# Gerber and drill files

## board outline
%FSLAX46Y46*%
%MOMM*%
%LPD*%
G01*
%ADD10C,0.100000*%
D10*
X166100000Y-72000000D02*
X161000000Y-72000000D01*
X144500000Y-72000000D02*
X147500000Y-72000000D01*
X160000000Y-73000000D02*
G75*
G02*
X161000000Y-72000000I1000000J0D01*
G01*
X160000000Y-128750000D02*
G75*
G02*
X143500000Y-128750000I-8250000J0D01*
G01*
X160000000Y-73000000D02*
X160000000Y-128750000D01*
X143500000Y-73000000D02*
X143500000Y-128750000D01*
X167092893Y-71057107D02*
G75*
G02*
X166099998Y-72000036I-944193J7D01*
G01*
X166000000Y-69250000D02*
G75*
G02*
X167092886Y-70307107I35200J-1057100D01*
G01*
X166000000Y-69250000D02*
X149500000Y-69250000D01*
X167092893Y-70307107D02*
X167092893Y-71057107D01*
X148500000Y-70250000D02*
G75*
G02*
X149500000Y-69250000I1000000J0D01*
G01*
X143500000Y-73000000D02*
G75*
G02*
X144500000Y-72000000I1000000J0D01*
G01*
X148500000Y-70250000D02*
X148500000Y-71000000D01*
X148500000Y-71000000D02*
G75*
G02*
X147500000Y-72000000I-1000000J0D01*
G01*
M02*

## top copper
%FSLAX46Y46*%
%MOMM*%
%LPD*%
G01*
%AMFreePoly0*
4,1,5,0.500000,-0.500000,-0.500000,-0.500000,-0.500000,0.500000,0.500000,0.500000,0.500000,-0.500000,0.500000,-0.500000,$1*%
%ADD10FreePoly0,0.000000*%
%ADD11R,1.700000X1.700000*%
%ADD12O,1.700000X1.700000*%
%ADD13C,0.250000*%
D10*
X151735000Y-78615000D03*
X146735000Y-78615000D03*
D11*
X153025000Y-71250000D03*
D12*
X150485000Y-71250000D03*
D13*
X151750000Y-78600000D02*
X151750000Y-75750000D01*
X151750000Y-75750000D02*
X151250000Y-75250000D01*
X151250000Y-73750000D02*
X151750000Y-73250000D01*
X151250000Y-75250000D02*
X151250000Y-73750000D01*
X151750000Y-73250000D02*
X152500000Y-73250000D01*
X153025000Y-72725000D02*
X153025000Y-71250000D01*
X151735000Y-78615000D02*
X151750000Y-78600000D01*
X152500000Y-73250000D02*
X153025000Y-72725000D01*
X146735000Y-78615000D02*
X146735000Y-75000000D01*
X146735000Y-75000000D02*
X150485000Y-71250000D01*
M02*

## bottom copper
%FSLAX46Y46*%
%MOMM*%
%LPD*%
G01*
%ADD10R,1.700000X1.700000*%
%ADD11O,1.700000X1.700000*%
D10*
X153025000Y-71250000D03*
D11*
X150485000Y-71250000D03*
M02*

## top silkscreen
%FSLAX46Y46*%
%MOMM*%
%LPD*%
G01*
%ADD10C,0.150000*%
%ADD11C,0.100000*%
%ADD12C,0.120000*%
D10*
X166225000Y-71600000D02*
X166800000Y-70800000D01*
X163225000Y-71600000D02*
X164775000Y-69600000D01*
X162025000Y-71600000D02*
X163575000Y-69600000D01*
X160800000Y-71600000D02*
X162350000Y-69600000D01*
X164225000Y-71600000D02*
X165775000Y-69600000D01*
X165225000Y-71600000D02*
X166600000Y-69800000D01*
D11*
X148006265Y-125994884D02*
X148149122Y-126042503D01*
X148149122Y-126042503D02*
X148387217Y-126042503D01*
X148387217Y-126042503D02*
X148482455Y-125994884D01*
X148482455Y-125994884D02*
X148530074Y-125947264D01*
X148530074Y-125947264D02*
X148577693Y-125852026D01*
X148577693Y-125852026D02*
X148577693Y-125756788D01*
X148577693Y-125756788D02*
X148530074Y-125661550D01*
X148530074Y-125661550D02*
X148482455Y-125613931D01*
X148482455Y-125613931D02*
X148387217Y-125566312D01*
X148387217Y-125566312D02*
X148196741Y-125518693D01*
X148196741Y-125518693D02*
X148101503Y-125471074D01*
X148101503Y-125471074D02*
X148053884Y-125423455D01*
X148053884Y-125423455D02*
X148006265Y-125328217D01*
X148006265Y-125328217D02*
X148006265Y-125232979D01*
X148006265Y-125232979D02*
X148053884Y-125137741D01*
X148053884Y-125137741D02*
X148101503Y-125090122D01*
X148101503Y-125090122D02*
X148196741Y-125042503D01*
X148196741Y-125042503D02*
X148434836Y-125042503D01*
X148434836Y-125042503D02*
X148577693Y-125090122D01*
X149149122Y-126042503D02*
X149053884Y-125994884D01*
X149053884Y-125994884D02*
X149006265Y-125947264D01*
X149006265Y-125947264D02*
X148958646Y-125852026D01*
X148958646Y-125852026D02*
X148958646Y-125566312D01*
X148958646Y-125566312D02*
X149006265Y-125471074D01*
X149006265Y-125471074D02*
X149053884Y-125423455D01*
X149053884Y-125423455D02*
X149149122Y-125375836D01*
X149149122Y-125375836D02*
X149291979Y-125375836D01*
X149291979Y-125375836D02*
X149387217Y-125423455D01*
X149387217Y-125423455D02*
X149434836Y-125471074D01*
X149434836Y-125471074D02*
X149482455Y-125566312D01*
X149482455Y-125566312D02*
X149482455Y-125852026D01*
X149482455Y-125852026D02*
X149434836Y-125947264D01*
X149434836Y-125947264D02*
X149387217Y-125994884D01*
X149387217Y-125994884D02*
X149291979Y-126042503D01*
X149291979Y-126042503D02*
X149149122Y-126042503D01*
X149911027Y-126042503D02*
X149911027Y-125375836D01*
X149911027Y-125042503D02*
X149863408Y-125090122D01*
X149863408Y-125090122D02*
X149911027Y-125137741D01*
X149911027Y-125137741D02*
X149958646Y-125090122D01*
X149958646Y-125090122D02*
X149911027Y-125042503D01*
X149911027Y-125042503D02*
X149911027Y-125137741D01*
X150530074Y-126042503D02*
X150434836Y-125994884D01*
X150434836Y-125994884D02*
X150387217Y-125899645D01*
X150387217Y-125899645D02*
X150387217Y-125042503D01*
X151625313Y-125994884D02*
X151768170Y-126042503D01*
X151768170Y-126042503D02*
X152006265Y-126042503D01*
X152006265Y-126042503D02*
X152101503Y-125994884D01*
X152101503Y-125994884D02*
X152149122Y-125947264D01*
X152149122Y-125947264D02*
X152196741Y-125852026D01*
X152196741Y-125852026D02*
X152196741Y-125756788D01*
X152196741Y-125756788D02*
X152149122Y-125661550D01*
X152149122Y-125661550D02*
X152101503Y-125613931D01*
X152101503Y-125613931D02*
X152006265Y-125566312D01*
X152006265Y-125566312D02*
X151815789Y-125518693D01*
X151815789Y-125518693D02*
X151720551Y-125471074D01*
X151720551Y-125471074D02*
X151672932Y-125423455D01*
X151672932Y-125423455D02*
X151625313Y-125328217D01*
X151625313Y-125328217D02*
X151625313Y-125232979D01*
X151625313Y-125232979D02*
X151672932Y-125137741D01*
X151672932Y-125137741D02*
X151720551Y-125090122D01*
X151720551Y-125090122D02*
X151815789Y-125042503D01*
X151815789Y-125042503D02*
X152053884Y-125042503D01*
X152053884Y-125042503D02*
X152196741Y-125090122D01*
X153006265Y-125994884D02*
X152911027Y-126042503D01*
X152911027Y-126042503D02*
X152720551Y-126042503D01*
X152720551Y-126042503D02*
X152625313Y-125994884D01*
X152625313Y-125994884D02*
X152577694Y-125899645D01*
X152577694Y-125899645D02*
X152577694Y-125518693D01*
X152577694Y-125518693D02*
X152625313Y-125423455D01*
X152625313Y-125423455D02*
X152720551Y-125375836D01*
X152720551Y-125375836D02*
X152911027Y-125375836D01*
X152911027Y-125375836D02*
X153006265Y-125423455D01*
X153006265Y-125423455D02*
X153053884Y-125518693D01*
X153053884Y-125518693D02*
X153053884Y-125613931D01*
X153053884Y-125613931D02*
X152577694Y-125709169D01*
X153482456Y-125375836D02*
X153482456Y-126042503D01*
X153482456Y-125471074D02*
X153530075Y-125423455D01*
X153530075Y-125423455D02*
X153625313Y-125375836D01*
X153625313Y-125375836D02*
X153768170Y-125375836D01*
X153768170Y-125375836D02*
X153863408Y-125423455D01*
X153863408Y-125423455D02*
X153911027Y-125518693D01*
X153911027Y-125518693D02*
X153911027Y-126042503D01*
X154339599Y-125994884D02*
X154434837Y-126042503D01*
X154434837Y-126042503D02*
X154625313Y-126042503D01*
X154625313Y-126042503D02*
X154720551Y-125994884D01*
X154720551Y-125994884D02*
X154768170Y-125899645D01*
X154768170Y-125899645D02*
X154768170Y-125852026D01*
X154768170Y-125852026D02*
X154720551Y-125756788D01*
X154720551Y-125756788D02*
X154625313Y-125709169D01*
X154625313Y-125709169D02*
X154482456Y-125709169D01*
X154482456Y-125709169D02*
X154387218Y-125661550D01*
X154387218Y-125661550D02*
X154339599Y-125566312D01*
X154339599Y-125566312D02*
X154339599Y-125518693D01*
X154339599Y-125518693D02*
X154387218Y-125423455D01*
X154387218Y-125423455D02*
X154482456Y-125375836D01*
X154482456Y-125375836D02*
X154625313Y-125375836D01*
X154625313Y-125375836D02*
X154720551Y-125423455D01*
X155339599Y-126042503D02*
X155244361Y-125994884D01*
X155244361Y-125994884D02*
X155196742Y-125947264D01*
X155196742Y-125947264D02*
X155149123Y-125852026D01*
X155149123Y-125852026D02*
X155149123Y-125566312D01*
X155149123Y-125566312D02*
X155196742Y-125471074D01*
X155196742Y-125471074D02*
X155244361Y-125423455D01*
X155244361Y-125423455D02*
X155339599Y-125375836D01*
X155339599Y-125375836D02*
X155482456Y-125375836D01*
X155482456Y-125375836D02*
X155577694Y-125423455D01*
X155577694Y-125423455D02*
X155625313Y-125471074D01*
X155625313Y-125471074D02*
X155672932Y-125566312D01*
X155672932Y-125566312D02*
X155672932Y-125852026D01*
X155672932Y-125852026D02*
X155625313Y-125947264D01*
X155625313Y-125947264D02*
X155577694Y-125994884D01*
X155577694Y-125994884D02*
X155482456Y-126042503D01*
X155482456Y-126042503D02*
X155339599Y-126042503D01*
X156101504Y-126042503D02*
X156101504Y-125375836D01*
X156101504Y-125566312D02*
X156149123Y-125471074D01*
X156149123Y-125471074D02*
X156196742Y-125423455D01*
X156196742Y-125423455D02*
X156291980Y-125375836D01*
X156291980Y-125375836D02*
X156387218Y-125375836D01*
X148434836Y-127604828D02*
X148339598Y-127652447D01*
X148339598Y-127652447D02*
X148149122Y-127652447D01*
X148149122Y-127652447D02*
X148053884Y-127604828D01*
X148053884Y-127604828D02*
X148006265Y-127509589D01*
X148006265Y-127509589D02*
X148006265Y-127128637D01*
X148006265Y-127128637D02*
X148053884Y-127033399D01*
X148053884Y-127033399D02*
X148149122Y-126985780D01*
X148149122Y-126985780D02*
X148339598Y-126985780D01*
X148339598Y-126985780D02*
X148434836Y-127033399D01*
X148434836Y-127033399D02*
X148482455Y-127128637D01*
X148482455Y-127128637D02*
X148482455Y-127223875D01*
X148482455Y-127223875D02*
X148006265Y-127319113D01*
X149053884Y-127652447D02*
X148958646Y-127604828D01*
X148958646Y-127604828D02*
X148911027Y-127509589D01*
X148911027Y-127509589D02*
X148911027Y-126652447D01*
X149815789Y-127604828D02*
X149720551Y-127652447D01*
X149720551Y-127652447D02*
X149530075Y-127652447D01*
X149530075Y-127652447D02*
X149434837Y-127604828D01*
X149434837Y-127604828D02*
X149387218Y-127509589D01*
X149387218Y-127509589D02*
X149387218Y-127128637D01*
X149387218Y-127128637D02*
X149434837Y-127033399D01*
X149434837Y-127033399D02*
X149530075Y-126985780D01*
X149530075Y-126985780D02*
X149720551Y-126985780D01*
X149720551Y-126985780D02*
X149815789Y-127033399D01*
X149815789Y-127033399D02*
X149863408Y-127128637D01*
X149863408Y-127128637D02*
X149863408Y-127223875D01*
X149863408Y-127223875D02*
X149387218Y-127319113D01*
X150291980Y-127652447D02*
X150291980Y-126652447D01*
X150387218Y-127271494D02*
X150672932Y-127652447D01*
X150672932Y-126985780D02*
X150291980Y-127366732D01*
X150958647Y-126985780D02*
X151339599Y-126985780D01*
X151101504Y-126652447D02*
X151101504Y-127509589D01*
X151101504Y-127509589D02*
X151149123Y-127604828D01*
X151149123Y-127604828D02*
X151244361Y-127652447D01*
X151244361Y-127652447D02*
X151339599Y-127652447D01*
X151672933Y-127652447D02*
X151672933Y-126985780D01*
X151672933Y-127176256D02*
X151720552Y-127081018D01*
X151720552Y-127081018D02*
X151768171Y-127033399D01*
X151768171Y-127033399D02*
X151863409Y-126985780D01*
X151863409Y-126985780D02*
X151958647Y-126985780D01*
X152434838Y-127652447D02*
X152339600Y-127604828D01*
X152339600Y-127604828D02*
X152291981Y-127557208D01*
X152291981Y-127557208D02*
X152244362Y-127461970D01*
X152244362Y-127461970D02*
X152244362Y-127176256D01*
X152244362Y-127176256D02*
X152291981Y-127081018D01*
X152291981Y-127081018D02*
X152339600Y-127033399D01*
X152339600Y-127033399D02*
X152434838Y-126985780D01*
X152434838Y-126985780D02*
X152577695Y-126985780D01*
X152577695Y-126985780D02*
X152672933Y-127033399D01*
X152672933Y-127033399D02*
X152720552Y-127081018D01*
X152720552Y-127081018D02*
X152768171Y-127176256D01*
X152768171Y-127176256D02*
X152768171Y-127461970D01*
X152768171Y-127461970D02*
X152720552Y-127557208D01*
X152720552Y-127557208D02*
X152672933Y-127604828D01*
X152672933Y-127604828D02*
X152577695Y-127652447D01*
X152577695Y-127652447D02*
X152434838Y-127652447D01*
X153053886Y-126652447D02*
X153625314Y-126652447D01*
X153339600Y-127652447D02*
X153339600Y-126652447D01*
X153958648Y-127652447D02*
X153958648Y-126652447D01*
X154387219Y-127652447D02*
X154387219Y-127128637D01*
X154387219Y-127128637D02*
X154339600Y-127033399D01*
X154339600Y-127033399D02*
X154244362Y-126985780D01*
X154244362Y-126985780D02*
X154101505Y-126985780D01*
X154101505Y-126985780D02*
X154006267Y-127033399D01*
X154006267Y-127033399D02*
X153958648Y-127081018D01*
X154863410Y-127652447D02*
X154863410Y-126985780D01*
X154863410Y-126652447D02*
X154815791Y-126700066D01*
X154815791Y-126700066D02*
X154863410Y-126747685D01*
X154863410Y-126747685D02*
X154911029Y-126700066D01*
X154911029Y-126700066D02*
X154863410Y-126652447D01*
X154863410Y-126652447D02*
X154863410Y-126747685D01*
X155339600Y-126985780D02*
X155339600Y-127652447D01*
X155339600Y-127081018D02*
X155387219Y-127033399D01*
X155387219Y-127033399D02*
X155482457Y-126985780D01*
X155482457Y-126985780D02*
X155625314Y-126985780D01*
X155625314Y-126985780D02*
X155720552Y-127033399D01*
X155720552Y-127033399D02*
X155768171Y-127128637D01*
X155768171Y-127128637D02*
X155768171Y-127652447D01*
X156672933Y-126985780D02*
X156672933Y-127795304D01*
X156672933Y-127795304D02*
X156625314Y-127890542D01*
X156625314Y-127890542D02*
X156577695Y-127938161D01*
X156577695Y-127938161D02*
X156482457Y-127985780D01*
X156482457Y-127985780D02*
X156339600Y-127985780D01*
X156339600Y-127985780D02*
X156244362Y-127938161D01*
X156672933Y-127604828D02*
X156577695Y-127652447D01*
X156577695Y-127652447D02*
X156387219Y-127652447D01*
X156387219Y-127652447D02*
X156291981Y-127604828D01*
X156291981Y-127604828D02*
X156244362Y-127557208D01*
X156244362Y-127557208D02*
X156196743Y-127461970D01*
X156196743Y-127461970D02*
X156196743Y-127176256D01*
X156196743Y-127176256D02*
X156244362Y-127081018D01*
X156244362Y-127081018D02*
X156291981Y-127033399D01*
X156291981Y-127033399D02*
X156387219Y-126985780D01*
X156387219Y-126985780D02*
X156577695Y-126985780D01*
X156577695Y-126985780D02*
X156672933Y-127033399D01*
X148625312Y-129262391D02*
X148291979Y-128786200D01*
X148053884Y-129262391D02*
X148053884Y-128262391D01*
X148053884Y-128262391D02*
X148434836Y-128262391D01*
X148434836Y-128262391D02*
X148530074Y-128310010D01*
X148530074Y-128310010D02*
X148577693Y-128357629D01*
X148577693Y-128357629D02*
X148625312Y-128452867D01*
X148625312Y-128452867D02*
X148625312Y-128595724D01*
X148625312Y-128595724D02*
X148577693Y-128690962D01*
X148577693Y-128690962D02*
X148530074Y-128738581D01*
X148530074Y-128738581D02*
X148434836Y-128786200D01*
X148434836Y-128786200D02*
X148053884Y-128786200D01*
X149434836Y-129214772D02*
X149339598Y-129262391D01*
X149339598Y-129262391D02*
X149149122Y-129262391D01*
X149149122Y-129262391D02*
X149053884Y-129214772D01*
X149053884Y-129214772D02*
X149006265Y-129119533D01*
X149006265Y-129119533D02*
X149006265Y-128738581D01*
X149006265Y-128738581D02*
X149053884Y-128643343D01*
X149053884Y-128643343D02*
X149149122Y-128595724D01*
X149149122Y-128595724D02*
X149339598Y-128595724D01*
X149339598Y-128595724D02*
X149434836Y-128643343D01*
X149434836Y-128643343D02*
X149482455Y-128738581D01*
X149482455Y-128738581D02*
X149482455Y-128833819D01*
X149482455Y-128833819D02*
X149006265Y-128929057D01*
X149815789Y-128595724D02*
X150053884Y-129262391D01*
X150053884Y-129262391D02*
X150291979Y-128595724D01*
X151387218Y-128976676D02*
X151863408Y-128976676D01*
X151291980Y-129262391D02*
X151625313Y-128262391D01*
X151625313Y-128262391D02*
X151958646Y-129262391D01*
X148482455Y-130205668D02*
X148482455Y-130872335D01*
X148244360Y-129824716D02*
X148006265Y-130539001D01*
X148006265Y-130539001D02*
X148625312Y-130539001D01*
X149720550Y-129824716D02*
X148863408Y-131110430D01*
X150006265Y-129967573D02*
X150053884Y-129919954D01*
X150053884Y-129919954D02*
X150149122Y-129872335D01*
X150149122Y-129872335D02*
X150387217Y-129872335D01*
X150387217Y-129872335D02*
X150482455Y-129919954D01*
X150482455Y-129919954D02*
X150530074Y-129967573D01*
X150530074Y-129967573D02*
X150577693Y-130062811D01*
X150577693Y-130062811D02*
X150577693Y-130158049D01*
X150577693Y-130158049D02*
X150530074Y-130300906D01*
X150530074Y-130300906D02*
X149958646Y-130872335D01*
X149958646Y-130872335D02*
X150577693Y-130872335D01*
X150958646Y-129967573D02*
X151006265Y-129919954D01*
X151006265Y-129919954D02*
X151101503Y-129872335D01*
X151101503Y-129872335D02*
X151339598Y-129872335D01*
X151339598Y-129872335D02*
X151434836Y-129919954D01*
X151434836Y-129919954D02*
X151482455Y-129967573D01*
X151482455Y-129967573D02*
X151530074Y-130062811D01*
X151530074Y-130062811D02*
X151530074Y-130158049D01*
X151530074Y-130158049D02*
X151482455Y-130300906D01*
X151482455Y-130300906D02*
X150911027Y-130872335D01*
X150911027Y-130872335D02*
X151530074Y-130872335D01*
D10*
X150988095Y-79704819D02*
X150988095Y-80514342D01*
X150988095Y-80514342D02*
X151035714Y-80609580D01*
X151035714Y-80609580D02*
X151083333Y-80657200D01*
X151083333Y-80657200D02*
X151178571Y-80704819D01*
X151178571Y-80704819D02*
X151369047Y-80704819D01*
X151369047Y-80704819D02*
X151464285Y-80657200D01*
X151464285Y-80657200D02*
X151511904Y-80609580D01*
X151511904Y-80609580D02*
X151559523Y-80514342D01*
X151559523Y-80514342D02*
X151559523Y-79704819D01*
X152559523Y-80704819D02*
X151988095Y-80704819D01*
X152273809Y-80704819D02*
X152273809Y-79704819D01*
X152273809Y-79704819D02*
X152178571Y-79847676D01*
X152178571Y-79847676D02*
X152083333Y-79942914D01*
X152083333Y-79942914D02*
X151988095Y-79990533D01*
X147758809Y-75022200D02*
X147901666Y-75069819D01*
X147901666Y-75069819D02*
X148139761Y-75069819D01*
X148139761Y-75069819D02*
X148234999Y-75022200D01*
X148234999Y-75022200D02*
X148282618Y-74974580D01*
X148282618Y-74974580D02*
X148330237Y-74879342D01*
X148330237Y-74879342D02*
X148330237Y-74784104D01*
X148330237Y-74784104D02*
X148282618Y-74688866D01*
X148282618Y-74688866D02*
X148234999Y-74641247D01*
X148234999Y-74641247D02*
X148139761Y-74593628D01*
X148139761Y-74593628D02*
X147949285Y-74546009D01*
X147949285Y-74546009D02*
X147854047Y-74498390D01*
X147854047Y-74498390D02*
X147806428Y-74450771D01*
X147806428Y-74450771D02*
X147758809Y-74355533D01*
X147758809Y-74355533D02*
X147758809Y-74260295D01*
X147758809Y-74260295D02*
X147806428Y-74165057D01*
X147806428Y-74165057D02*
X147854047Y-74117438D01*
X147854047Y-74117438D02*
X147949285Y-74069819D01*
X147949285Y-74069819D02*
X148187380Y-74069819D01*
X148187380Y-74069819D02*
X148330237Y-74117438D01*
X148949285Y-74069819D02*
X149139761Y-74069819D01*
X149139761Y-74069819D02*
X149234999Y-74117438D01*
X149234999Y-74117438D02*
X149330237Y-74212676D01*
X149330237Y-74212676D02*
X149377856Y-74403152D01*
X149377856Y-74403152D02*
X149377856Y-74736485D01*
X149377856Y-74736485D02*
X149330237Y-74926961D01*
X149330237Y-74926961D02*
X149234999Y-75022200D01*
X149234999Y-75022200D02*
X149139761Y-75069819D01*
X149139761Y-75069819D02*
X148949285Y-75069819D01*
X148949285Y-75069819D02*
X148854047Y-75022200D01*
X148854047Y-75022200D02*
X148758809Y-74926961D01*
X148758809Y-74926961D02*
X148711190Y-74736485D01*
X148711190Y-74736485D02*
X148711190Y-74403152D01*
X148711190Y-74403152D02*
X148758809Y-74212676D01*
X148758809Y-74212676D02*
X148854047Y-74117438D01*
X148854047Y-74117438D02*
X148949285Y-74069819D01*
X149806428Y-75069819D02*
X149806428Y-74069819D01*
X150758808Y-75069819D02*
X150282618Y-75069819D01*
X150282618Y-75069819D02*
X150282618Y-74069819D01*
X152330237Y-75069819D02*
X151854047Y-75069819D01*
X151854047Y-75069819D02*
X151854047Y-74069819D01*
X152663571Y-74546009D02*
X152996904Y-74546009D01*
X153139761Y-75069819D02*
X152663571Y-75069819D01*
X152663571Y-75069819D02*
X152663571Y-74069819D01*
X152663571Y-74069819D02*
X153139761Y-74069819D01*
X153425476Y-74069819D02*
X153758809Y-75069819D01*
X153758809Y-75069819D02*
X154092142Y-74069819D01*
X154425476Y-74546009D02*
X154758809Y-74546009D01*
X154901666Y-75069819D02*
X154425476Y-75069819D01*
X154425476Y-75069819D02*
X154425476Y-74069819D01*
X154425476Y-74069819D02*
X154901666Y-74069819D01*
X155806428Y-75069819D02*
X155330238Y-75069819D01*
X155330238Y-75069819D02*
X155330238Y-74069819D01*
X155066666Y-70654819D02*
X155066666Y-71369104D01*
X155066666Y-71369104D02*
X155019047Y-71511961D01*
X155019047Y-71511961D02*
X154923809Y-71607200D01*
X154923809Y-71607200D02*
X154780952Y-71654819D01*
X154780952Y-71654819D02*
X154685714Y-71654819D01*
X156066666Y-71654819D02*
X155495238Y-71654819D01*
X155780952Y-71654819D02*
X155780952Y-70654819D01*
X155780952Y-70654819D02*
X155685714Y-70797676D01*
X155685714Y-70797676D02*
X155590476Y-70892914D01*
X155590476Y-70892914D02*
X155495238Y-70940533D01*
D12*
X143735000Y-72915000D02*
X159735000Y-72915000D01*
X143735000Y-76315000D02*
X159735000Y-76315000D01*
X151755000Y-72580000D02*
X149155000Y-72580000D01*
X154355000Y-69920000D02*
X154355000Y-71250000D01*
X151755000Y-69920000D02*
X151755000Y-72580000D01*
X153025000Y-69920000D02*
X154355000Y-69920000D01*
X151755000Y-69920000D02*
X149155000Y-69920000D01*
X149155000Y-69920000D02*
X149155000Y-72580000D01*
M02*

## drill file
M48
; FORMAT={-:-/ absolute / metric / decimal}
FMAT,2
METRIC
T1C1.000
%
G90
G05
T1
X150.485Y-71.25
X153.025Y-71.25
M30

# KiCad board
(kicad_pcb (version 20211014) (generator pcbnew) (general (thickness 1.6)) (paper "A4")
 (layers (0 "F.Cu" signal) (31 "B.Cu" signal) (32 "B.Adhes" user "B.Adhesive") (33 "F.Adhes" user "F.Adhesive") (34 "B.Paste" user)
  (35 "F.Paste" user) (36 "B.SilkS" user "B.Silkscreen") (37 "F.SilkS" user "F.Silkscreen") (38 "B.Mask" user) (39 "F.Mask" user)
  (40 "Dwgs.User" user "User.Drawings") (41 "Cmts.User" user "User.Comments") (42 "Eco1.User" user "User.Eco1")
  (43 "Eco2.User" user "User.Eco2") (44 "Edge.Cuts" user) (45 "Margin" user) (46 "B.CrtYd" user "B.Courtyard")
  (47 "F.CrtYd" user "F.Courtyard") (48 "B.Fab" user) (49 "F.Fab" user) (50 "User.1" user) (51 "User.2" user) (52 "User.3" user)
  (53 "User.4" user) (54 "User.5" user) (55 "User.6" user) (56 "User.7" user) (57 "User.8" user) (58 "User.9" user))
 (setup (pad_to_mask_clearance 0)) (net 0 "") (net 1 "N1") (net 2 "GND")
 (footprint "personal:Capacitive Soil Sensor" (layer "F.Cu") (at 151.735 78.615)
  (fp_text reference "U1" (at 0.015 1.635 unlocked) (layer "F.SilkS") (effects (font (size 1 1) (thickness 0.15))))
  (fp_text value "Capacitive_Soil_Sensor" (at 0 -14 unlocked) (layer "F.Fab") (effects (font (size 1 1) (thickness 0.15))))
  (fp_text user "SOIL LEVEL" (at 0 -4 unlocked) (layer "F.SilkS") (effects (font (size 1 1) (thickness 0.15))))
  (fp_line (start -8 -5.7) (end 8 -5.7) (layer "F.SilkS") (width 0.12))
  (fp_line (start -8 -2.3) (end 8 -2.3) (layer "F.SilkS") (width 0.12))
  (pad "1" smd custom (at 0 0) (size 1 1) (layers "F.Cu") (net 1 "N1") (options (clearance outline) (anchor rect)) (primitives))
  (pad "2" smd custom (at -5 0) (size 1 1) (layers "F.Cu") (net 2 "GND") (options (clearance outline) (anchor rect)) (primitives)))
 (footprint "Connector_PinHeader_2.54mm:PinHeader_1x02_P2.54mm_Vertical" (layer "F.Cu") (at 153.025 71.25 -90)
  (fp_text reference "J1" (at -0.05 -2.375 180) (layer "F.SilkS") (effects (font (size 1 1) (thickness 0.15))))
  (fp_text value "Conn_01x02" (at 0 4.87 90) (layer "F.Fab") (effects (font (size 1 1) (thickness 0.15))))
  (fp_line (start 1.33 1.27) (end 1.33 3.87) (layer "F.SilkS") (width 0.12))
  (fp_line (start -1.33 -1.33) (end 0 -1.33) (layer "F.SilkS") (width 0.12))
  (fp_line (start -1.33 1.27) (end 1.33 1.27) (layer "F.SilkS") (width 0.12))
  (fp_line (start -1.33 0) (end -1.33 -1.33) (layer "F.SilkS") (width 0.12))
  (fp_line (start -1.33 1.27) (end -1.33 3.87) (layer "F.SilkS") (width 0.12))
  (fp_line (start -1.33 3.87) (end 1.33 3.87) (layer "F.SilkS") (width 0.12))
  (pad "1" thru_hole rect locked (at 0 0 270) (size 1.7 1.7) (drill 1) (layers *.Cu *.Mask) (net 1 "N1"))
  (pad "2" thru_hole oval locked (at 0 2.54 270) (size 1.7 1.7) (drill 1) (layers *.Cu *.Mask) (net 2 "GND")))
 (gr_line (start 166.225 71.6) (end 166.8 70.8) (layer "F.SilkS") (width 0.15))
 (gr_line (start 163.225 71.6) (end 164.775 69.6) (layer "F.SilkS") (width 0.15))
 (gr_line (start 162.025 71.6) (end 163.575 69.6) (layer "F.SilkS") (width 0.15))
 (gr_line (start 160.8 71.6) (end 162.35 69.6) (layer "F.SilkS") (width 0.15))
 (gr_line (start 164.225 71.6) (end 165.775 69.6) (layer "F.SilkS") (width 0.15))
 (gr_line (start 165.225 71.6) (end 166.6 69.8) (layer "F.SilkS") (width 0.15))
 (gr_line (start 166.1 72) (end 161 72) (layer "Edge.Cuts") (width 0.1))
 (gr_line (start 144.5 72) (end 147.5 72) (layer "Edge.Cuts") (width 0.1))
 (gr_arc (start 160 73) (mid 160.292893 72.292893) (end 161 72) (layer "Edge.Cuts") (width 0.1))
 (gr_arc (start 160 128.75) (mid 151.75 137) (end 143.5 128.75) (layer "Edge.Cuts") (width 0.1))
 (gr_line (start 160 73) (end 160 128.75) (layer "Edge.Cuts") (width 0.1))
 (gr_line (start 143.5 73) (end 143.5 128.75) (layer "Edge.Cuts") (width 0.1))
 (gr_arc (start 167.092893 71.057107) (mid 166.798893 71.741736) (end 166.1 72) (layer "Edge.Cuts") (width 0.1))
 (gr_arc (start 166 69.25) (mid 166.770552 69.546861) (end 167.092893 70.307107) (layer "Edge.Cuts") (width 0.1))
 (gr_line (start 166 69.25) (end 149.5 69.25) (layer "Edge.Cuts") (width 0.1))
 (gr_line (start 167.092893 70.307107) (end 167.092893 71.057107) (layer "Edge.Cuts") (width 0.1))
 (gr_arc (start 148.5 70.25) (mid 148.792893 69.542893) (end 149.5 69.25) (layer "Edge.Cuts") (width 0.1))
 (gr_arc (start 143.5 73) (mid 143.792893 72.292893) (end 144.5 72) (layer "Edge.Cuts") (width 0.1))
 (gr_line (start 148.5 70.25) (end 148.5 71) (layer "Edge.Cuts") (width 0.1))
 (gr_arc (start 148.5 71) (mid 148.207107 71.707107) (end 147.5 72) (layer "Edge.Cuts") (width 0.1))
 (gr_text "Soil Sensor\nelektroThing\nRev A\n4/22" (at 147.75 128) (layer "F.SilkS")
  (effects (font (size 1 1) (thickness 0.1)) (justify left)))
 (segment (start 151.75 78.6) (end 151.75 75.75) (width 0.25) (layer "F.Cu") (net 1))
 (segment (start 151.75 75.75) (end 151.25 75.25) (width 0.25) (layer "F.Cu") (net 1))
 (segment (start 151.25 73.75) (end 151.75 73.25) (width 0.25) (layer "F.Cu") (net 1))
 (segment (start 151.25 75.25) (end 151.25 73.75) (width 0.25) (layer "F.Cu") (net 1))
 (segment (start 151.75 73.25) (end 152.5 73.25) (width 0.25) (layer "F.Cu") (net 1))
 (segment (start 153.025 72.725) (end 153.025 71.25) (width 0.25) (layer "F.Cu") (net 1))
 (segment (start 151.735 78.615) (end 151.75 78.6) (width 0.25) (layer "F.Cu") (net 1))
 (segment (start 152.5 73.25) (end 153.025 72.725) (width 0.25) (layer "F.Cu") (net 1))
 (segment (start 146.735 78.615) (end 146.735 75) (width 0.25) (layer "F.Cu") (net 2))
 (segment (start 146.735 75) (end 150.485 71.25) (width 0.25) (layer "F.Cu") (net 2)))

